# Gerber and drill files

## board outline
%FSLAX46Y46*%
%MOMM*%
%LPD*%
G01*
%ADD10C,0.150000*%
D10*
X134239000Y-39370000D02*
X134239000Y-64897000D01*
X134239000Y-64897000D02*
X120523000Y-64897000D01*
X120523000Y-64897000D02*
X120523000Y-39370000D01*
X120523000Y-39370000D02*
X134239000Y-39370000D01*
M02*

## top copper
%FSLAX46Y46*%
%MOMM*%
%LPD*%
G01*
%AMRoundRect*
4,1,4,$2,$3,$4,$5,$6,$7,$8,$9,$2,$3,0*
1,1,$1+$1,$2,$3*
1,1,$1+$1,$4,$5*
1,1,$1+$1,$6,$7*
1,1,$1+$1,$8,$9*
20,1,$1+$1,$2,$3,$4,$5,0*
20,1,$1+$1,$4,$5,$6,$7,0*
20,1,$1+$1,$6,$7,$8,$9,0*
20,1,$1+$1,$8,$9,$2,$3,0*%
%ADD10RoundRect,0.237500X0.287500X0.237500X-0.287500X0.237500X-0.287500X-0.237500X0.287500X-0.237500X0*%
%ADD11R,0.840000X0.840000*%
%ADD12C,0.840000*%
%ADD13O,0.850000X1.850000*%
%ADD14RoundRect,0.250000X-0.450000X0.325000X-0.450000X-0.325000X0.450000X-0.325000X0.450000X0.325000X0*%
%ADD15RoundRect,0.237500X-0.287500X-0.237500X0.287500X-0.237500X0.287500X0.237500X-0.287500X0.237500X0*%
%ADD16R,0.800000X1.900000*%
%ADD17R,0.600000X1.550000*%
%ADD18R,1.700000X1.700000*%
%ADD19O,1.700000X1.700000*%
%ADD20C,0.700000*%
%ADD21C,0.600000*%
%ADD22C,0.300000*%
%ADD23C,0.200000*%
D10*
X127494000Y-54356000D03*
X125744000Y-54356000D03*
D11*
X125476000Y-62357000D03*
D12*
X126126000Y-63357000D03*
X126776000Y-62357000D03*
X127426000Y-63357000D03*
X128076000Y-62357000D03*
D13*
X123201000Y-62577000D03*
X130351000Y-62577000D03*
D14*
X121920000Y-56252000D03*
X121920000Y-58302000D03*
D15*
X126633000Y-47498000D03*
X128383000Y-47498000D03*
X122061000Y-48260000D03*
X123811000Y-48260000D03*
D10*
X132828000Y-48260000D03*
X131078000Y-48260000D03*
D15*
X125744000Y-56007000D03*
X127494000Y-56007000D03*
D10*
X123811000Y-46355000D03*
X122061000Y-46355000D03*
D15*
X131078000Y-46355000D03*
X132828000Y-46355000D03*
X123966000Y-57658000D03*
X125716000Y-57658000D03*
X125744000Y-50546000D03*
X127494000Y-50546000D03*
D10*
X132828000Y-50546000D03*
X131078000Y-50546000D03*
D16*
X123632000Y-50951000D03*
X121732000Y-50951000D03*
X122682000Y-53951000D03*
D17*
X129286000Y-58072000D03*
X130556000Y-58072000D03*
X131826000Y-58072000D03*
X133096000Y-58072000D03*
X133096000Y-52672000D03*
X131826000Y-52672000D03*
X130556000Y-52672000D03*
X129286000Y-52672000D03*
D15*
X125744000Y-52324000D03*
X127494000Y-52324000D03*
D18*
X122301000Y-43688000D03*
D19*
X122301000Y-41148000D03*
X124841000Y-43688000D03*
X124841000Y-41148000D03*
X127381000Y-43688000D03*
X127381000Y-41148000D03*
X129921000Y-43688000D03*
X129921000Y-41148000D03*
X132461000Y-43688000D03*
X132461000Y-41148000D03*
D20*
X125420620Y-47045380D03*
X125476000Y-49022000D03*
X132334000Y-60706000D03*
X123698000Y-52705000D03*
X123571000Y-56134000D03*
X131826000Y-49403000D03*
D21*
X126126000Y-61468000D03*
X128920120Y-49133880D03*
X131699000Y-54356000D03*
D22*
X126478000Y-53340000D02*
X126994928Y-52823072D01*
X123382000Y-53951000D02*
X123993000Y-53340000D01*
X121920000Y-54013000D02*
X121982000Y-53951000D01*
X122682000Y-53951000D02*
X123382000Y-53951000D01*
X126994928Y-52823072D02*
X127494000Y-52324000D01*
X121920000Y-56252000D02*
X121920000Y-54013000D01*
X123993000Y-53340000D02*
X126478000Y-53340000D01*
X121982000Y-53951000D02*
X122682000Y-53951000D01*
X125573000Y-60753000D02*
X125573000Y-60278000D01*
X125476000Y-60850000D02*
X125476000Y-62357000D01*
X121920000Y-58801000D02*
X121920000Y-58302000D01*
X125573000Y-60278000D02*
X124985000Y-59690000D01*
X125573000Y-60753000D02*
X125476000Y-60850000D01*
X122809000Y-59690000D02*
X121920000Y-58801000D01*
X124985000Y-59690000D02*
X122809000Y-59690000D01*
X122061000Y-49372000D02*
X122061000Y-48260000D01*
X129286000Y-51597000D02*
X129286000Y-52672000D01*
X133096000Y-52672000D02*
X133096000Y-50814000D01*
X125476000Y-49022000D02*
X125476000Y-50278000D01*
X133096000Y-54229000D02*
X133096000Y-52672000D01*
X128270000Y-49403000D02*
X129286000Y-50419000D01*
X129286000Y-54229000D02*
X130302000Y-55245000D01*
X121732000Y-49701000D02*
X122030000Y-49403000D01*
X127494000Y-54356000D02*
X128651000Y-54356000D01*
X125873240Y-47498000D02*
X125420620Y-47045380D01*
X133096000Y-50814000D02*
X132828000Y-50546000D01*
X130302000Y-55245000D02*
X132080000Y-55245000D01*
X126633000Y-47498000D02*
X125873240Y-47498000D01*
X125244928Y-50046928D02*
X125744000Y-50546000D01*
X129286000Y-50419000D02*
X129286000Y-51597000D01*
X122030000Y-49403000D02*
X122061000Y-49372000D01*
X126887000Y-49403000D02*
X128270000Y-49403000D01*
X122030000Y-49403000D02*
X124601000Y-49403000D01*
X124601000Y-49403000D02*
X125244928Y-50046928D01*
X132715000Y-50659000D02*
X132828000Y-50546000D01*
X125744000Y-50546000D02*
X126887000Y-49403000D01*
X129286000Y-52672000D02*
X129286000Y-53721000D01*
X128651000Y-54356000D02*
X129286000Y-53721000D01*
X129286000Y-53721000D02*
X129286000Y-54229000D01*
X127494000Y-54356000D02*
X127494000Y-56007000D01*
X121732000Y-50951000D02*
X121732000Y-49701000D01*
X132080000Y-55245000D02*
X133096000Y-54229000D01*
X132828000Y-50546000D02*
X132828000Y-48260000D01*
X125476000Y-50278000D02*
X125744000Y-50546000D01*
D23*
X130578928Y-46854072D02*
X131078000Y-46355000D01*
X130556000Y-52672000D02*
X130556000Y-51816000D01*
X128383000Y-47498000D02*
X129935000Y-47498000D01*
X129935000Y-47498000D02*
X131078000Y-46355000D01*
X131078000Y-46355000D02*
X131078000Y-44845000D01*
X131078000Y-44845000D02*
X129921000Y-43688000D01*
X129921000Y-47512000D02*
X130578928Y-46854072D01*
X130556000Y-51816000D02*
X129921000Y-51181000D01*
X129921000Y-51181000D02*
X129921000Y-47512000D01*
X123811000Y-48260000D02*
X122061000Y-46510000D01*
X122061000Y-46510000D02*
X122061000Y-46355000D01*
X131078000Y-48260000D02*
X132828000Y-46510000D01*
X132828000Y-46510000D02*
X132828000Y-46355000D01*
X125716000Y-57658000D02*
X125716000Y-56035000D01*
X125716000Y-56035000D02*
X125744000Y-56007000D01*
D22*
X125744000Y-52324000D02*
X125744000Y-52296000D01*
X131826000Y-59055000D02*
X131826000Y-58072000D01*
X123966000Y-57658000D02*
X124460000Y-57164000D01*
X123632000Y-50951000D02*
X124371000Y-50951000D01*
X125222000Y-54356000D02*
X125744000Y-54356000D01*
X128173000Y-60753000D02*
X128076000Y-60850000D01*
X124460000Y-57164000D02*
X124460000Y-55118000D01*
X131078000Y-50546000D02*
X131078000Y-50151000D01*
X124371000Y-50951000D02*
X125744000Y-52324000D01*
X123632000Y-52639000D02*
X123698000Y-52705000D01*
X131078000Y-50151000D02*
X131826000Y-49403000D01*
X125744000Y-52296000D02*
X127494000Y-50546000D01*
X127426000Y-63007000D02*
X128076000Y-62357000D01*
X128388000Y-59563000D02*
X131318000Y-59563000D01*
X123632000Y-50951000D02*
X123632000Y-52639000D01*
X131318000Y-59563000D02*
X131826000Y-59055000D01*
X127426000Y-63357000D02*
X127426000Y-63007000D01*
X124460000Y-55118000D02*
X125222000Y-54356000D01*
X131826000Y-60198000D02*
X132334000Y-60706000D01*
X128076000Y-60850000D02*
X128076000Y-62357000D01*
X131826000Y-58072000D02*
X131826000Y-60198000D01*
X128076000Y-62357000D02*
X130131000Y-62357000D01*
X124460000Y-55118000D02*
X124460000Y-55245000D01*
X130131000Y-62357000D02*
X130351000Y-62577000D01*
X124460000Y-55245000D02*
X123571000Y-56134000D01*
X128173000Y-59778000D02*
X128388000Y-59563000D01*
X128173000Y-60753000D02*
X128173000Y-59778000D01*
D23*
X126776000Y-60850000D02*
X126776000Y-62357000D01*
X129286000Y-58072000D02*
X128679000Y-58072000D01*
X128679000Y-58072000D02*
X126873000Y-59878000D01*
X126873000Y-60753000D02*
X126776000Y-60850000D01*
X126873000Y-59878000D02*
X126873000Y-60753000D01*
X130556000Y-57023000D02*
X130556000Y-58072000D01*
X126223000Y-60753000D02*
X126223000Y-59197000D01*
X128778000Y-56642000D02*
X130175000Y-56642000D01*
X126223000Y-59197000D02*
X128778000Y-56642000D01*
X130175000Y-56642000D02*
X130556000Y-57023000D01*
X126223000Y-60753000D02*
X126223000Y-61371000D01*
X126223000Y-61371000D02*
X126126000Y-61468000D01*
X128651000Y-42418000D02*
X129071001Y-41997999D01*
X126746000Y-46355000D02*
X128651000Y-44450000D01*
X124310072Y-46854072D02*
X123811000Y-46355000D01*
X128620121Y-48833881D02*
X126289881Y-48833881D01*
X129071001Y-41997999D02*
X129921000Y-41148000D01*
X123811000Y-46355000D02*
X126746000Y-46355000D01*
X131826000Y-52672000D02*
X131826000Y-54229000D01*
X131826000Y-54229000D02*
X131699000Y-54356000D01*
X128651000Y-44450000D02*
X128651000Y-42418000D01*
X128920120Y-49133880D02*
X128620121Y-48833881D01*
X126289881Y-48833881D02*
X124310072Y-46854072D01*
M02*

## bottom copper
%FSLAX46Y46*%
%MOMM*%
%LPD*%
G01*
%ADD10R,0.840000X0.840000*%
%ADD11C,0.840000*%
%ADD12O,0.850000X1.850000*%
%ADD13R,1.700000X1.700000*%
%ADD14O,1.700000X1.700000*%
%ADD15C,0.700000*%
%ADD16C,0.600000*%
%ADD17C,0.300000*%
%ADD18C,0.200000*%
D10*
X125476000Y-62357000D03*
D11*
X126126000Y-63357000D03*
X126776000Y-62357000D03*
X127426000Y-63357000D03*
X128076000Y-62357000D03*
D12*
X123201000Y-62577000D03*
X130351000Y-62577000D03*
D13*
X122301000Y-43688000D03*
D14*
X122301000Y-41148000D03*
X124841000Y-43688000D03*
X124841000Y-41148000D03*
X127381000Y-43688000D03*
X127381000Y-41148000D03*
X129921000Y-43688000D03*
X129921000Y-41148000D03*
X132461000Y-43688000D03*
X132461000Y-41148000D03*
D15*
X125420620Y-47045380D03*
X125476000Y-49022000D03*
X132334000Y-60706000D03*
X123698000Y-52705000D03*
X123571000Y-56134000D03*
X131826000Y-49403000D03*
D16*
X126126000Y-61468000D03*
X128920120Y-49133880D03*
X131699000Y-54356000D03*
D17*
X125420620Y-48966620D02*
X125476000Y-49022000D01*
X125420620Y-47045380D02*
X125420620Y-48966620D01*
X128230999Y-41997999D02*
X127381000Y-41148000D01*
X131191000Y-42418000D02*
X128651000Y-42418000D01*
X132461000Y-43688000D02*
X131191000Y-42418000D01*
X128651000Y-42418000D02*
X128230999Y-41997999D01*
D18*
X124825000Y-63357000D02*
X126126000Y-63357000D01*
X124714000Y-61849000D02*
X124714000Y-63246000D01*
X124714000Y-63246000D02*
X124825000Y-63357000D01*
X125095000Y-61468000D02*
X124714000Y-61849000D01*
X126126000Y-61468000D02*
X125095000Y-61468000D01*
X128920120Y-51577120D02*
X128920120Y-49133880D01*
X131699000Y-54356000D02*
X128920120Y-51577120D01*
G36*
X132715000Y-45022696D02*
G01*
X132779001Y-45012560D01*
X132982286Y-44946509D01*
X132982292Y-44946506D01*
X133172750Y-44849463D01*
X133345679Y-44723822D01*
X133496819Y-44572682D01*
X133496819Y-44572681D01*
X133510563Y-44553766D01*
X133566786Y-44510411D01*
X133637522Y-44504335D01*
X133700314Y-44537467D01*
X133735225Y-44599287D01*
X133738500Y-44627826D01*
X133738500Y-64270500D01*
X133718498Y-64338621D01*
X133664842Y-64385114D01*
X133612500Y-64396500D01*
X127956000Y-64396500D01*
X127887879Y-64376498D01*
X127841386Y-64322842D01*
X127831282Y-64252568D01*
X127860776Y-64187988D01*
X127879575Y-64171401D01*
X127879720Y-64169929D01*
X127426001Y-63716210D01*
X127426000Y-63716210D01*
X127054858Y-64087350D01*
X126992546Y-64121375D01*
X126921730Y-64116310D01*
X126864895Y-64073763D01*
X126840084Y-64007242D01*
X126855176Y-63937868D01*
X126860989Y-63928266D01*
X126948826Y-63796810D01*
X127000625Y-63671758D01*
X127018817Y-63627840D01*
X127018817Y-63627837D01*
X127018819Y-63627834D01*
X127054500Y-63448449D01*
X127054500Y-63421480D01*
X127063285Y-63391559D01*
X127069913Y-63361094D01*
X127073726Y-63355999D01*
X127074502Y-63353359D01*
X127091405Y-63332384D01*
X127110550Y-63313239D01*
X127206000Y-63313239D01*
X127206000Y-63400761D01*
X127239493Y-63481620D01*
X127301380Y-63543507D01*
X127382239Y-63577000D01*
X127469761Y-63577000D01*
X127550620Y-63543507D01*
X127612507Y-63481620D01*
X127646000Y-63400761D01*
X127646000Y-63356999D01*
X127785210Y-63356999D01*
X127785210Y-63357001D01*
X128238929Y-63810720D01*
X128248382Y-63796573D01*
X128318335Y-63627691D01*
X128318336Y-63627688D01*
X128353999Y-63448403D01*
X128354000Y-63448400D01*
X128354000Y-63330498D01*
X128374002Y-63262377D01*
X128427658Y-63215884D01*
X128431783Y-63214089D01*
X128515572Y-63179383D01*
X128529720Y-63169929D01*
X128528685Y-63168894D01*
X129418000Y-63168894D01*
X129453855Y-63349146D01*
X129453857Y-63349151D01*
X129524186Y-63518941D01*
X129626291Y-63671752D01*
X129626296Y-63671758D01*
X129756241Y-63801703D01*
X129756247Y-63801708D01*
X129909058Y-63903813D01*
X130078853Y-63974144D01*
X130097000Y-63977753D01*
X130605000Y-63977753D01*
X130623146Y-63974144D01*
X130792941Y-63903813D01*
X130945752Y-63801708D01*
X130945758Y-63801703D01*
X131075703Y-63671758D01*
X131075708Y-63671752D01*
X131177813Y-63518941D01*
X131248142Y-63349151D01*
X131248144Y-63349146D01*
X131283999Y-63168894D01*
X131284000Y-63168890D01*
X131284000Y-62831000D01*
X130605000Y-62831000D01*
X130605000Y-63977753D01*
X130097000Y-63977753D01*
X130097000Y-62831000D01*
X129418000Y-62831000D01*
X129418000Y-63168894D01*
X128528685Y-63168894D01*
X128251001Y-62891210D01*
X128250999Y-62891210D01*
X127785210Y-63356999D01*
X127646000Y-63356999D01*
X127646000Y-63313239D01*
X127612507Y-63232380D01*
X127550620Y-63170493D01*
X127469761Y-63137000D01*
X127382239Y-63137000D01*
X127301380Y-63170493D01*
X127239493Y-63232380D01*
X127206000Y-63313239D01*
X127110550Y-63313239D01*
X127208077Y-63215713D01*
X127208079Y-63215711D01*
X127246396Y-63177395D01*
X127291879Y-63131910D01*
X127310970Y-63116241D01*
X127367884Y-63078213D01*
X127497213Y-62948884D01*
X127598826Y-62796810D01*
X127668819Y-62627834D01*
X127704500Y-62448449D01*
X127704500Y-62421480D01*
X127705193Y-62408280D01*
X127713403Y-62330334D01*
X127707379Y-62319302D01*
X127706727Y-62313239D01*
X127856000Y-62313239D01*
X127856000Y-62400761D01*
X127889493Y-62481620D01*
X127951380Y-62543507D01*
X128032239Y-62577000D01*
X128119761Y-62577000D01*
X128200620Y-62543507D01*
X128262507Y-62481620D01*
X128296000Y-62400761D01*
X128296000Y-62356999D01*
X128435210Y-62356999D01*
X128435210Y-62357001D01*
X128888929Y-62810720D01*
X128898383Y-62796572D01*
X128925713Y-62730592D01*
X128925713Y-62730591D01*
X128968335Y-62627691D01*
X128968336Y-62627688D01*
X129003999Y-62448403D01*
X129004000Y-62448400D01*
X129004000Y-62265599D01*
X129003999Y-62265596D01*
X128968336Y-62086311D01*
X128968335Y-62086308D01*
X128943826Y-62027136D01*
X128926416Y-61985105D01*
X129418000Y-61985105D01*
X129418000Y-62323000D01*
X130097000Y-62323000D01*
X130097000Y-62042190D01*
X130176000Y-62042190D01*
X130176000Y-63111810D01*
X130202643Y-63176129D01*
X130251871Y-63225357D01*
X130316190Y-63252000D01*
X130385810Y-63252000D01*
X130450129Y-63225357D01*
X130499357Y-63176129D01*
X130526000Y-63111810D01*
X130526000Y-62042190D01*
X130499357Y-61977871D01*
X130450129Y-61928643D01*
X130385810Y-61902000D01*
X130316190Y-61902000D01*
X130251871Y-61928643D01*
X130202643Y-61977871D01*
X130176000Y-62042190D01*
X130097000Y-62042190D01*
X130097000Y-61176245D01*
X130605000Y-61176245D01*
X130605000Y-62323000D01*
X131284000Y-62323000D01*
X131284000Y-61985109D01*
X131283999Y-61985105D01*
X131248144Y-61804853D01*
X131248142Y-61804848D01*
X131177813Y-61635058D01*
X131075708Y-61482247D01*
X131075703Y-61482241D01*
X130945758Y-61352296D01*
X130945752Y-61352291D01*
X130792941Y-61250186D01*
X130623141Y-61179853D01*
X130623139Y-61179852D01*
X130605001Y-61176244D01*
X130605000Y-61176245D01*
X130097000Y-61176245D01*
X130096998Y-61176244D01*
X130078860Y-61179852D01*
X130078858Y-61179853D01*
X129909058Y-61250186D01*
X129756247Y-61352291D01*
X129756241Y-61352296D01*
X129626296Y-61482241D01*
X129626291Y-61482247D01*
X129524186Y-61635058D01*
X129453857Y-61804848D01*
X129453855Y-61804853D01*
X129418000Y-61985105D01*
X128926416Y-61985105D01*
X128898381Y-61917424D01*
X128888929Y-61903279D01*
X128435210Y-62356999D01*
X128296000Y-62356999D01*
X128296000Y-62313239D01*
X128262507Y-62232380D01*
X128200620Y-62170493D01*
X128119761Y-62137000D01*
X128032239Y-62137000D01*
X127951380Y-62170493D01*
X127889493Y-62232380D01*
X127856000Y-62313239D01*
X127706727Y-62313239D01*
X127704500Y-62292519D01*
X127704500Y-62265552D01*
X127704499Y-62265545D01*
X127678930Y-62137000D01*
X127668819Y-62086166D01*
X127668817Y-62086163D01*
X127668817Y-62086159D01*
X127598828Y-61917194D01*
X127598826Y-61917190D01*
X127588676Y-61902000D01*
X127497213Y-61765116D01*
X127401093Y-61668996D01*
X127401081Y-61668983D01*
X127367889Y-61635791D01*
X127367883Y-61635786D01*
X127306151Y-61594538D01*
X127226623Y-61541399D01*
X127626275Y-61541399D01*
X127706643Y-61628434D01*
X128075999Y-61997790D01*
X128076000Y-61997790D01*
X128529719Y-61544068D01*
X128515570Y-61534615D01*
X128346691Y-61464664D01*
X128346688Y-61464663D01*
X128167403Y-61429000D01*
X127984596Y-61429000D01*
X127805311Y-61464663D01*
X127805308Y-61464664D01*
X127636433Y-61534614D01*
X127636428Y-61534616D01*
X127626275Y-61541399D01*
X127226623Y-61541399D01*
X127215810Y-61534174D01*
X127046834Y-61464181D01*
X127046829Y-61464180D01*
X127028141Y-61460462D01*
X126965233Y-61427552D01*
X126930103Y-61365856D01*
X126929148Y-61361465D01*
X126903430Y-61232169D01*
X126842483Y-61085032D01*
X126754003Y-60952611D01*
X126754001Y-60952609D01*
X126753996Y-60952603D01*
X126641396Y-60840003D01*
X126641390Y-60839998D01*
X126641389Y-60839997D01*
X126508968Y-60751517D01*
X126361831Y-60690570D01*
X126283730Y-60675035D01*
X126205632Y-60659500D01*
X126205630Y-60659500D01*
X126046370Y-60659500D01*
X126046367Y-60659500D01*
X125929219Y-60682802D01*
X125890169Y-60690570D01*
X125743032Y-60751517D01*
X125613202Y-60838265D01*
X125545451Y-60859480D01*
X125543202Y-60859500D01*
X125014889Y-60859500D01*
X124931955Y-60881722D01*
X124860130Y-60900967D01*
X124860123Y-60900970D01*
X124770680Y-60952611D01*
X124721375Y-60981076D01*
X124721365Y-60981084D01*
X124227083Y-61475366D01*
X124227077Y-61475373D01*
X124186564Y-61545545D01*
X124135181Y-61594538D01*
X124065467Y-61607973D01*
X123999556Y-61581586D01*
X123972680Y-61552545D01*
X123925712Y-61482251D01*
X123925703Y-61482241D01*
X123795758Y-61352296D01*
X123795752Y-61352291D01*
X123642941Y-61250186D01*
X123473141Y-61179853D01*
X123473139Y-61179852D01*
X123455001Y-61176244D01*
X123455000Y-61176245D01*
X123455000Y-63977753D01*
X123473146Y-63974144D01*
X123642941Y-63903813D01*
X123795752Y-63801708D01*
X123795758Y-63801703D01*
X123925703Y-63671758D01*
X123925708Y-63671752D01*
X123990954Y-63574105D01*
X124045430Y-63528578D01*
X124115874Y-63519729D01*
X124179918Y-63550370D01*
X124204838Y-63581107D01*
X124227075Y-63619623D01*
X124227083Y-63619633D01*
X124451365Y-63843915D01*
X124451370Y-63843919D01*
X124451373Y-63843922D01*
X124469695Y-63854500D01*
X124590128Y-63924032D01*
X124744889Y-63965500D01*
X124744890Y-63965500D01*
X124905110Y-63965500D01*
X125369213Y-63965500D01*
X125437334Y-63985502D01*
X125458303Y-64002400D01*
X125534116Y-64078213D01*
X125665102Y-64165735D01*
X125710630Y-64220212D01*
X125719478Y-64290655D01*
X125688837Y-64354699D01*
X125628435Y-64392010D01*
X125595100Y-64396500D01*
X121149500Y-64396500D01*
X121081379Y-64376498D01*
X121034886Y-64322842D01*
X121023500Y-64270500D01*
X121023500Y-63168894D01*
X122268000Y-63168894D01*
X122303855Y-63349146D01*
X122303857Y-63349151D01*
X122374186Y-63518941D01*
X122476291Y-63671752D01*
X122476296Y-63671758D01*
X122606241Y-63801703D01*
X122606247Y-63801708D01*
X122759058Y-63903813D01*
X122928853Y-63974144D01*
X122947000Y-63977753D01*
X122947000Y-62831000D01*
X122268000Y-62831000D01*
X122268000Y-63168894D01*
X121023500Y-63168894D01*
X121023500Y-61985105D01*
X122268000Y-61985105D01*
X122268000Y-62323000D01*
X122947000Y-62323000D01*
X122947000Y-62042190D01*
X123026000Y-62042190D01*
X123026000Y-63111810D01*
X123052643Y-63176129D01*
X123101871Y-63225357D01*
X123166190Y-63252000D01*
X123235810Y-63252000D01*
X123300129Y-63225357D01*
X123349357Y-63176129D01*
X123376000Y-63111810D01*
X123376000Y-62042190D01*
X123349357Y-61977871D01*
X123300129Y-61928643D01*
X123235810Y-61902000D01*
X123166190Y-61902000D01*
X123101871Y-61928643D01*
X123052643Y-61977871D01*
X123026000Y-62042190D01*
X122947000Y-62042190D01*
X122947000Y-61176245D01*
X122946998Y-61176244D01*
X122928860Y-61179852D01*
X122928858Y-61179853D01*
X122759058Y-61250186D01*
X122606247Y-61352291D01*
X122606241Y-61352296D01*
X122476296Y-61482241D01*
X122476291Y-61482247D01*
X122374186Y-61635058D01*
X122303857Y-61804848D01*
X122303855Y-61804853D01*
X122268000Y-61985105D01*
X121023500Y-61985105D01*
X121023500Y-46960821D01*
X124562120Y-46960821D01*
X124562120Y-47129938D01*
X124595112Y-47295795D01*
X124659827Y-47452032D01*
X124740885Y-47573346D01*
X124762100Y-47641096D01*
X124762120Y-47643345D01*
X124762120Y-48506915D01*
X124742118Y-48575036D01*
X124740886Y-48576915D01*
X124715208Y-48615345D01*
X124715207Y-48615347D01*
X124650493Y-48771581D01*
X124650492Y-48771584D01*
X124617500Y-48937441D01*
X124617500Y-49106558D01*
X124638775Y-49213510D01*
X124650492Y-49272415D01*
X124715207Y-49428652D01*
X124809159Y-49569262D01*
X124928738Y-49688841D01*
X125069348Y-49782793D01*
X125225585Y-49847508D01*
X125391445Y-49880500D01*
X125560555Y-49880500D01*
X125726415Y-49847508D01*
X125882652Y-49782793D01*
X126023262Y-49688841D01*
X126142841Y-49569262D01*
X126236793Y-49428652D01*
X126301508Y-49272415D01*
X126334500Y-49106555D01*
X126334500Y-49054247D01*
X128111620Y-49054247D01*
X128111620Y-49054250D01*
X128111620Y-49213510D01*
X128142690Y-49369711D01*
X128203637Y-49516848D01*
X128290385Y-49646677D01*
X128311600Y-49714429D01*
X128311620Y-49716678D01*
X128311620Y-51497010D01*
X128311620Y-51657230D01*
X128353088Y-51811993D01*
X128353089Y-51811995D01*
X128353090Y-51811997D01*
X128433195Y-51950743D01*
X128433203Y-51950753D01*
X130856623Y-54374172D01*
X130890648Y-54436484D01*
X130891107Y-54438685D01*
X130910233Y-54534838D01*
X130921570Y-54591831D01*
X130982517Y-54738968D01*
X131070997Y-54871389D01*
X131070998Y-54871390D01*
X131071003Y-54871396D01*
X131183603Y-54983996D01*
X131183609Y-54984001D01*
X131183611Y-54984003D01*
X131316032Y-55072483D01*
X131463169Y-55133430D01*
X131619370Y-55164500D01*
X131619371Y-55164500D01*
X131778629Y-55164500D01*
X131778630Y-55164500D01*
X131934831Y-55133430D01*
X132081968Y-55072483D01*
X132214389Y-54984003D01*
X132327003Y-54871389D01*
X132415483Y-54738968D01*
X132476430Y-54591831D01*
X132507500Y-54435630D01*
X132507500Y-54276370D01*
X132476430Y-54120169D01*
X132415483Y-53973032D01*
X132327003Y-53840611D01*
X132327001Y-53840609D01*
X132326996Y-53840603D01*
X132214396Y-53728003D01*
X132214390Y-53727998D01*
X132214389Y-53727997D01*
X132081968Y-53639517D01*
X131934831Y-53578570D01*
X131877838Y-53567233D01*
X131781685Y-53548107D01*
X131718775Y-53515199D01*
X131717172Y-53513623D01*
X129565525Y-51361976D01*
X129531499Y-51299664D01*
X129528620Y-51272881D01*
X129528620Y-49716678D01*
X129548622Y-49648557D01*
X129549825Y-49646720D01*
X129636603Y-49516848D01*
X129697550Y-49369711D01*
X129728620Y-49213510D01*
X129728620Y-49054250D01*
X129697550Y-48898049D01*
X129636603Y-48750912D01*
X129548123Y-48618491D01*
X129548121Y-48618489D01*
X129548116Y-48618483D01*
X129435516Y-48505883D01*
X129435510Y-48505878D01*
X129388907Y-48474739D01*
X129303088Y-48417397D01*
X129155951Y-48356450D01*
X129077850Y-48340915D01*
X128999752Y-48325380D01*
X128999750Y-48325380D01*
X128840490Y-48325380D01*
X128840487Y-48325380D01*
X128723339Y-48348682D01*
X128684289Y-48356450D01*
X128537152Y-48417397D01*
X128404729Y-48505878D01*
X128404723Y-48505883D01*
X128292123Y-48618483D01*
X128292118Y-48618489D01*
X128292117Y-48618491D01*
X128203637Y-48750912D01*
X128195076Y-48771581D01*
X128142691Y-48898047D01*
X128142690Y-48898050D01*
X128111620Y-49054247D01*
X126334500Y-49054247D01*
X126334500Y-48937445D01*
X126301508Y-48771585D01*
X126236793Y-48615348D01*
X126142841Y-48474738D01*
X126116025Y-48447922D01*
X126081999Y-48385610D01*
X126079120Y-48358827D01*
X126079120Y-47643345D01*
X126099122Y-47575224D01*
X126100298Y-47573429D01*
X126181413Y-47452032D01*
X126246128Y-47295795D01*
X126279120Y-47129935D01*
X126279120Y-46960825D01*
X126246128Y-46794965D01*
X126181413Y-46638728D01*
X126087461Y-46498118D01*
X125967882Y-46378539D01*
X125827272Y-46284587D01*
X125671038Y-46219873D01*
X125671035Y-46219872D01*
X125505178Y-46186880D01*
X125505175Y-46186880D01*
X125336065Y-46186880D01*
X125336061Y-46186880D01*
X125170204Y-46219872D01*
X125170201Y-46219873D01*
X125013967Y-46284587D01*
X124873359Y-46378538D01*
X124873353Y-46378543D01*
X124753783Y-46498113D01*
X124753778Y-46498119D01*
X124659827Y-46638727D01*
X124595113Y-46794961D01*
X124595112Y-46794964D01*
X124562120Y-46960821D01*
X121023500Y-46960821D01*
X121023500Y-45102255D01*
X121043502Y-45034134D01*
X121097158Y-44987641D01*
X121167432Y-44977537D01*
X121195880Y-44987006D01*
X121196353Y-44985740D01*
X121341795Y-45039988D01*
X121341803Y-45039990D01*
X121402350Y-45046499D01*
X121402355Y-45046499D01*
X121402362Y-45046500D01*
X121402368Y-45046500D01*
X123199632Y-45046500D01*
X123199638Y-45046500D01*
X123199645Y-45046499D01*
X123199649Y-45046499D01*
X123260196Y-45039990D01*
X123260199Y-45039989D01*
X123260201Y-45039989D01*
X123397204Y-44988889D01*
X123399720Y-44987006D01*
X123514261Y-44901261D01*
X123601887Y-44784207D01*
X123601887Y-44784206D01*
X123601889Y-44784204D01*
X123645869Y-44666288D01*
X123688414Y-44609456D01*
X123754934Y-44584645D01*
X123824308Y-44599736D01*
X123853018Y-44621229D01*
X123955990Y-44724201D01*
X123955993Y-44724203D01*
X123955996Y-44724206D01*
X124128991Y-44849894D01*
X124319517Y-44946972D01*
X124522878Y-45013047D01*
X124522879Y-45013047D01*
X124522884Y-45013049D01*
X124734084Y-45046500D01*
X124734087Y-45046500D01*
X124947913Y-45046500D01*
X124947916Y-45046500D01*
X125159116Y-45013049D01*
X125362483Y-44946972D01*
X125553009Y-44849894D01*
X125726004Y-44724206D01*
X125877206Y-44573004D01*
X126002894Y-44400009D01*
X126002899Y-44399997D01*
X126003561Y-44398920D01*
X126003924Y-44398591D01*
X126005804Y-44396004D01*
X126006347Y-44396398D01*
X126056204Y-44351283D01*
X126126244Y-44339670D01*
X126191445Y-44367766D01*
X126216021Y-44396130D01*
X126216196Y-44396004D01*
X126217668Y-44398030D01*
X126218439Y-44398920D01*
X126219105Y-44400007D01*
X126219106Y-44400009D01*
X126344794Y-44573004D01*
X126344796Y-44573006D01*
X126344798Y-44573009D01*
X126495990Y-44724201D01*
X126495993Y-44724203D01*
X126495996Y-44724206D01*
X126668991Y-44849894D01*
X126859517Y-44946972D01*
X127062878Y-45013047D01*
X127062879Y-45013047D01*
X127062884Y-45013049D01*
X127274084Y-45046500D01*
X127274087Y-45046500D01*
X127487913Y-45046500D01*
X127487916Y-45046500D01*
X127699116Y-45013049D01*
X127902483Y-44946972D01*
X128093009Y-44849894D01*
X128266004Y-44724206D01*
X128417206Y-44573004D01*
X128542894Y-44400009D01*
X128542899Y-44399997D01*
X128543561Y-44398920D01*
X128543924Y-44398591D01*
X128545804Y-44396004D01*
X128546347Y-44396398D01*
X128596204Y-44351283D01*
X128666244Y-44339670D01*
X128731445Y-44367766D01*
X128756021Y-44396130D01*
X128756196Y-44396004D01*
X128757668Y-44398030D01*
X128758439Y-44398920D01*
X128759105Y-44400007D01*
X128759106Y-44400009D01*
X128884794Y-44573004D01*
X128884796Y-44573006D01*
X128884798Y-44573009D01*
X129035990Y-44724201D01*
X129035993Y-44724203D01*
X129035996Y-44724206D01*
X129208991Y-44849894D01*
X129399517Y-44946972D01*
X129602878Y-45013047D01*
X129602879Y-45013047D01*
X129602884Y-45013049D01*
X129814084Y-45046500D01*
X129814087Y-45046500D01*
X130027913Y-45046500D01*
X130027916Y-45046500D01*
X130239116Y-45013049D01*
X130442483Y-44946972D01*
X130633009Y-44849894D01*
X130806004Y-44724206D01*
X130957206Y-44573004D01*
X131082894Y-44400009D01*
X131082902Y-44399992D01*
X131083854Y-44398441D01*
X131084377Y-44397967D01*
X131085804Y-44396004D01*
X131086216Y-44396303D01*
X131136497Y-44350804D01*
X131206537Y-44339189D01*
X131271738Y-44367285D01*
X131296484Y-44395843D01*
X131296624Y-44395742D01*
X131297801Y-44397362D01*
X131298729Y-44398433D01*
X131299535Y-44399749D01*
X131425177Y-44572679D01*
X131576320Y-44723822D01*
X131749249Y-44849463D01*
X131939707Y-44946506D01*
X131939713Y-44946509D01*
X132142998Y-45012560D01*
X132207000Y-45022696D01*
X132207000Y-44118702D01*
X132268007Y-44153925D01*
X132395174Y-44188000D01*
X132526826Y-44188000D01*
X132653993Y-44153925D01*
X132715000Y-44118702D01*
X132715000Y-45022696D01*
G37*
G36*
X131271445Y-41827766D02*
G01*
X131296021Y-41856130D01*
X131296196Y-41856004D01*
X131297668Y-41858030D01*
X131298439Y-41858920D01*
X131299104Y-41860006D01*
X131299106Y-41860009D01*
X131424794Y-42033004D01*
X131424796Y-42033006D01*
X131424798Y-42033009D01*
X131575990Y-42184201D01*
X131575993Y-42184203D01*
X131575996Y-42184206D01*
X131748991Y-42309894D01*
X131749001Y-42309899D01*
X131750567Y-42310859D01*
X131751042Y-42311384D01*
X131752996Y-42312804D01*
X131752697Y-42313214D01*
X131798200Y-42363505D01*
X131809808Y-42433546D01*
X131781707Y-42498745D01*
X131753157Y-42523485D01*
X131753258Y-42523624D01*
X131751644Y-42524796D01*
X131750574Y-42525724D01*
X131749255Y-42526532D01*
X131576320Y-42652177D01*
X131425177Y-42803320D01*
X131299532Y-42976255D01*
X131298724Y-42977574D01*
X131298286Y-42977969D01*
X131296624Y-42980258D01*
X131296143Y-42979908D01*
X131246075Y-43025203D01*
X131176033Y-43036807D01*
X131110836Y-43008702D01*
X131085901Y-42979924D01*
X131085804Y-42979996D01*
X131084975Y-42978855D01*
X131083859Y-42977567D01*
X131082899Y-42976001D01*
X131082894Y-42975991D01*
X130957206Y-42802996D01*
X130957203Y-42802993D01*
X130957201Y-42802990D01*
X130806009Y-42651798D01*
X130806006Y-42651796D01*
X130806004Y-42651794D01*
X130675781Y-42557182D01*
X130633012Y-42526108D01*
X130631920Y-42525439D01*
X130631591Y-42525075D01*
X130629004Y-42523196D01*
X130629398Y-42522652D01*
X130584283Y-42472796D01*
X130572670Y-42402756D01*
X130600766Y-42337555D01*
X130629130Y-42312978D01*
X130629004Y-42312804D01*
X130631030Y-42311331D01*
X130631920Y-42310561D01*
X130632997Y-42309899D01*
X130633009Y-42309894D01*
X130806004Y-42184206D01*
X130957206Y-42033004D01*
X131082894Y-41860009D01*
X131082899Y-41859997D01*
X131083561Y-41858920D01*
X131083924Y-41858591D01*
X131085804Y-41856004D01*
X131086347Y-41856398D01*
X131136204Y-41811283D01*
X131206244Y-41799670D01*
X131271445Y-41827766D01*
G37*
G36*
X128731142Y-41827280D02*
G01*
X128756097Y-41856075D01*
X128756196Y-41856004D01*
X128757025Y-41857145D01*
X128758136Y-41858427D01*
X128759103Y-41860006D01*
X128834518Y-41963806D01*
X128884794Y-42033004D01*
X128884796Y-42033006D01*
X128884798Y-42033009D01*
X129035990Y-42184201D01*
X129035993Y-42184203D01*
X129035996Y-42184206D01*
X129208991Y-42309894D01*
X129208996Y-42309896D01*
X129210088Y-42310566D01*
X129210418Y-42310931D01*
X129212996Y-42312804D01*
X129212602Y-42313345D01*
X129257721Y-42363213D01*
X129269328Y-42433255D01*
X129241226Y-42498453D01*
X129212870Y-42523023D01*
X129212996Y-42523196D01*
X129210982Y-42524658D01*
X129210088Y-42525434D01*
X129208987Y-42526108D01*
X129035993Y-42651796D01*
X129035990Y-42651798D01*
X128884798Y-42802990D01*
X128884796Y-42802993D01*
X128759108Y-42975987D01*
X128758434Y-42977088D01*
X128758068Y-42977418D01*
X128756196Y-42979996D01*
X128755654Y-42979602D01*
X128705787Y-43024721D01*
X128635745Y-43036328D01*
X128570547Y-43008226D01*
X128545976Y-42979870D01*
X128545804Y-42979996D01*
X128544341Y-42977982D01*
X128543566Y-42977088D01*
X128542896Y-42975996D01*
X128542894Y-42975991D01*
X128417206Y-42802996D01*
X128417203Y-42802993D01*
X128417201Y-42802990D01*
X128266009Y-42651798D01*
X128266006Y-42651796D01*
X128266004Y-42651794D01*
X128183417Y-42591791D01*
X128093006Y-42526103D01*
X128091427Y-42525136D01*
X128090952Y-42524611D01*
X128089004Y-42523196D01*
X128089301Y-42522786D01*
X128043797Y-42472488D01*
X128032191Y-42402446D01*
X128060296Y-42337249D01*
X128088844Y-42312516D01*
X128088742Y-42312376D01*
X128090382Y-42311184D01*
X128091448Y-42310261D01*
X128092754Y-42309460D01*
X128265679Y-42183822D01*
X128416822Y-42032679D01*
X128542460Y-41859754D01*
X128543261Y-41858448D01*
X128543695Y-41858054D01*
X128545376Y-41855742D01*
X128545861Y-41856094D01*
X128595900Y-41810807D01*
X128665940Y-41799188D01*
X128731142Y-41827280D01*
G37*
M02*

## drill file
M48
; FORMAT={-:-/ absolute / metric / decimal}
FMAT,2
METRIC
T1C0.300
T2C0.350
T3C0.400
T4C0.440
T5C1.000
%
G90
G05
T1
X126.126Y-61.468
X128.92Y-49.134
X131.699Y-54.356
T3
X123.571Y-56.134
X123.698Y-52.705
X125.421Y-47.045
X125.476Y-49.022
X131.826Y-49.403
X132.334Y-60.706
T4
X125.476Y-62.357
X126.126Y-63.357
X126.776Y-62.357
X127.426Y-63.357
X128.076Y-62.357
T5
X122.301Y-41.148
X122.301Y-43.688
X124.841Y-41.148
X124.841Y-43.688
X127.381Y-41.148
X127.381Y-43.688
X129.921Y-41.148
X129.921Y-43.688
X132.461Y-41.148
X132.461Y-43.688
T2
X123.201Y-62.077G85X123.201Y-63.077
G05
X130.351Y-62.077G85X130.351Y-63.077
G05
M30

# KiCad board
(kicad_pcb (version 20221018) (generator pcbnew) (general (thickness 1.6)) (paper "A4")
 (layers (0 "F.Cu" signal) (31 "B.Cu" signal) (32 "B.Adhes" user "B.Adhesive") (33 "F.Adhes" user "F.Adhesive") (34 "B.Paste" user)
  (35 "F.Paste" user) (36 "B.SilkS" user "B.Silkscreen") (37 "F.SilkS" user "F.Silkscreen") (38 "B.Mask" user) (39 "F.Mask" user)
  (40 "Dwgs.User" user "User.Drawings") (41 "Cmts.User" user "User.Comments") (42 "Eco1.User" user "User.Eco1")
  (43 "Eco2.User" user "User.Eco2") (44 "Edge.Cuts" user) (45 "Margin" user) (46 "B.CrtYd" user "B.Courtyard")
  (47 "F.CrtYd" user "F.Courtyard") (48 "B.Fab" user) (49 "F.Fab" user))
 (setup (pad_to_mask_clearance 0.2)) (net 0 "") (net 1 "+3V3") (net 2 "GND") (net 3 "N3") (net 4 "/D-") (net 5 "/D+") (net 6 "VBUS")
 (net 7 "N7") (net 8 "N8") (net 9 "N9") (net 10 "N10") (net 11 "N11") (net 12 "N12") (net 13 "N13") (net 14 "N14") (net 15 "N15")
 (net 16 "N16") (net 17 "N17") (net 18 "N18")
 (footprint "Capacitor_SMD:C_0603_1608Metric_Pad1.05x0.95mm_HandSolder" (layer "F.Cu") (at 126.619 54.356 180)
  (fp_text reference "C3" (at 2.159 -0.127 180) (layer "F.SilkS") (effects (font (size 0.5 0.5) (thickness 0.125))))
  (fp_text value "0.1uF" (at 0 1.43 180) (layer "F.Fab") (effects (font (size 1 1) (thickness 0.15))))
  (pad "1" smd roundrect (at -0.875 0 180) (size 1.05 0.95) (layers "F.Cu" "F.Paste" "F.Mask") (roundrect_rratio 0.25) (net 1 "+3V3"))
  (pad "2" smd roundrect (at 0.875 0 180) (size 1.05 0.95) (layers "F.Cu" "F.Paste" "F.Mask") (roundrect_rratio 0.25) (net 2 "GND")))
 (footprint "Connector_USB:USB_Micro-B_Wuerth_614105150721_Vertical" (layer "F.Cu") (at 125.476 62.357)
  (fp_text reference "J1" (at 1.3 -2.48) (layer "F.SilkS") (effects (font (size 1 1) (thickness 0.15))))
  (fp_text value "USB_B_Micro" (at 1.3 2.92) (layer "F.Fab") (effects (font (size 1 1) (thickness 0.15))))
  (pad "1" thru_hole rect (at 0 0) (size 0.84 0.84) (drill 0.44) (layers "*.Cu" "*.Mask") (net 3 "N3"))
  (pad "2" thru_hole circle (at 0.65 1) (size 0.84 0.84) (drill 0.44) (layers "*.Cu" "*.Mask") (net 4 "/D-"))
  (pad "3" thru_hole circle (at 1.3 0) (size 0.84 0.84) (drill 0.44) (layers "*.Cu" "*.Mask") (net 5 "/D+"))
  (pad "4" thru_hole circle (at 1.95 1) (size 0.84 0.84) (drill 0.44) (layers "*.Cu" "*.Mask") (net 2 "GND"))
  (pad "5" thru_hole circle (at 2.6 0) (size 0.84 0.84) (drill 0.44) (layers "*.Cu" "*.Mask") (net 2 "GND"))
  (pad "6" thru_hole oval (at -2.275 0.22) (size 0.85 1.85) (drill oval 0.35 1.35) (layers "*.Cu" "*.Mask") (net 2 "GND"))
  (pad "6" thru_hole oval (at 4.875 0.22) (size 0.85 1.85) (drill oval 0.35 1.35) (layers "*.Cu" "*.Mask") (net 2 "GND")))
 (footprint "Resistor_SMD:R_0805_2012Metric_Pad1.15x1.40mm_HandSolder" (layer "F.Cu") (at 121.92 57.277 -90)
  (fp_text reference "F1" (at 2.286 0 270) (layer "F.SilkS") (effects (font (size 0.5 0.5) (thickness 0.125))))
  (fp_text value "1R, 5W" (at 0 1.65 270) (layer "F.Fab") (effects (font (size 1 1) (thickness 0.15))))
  (pad "1" smd roundrect (at -1.025 0 270) (size 1.15 1.4) (layers "F.Cu" "F.Paste" "F.Mask") (roundrect_rratio 0.217391) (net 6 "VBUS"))
  (pad "2" smd roundrect (at 1.025 0 270) (size 1.15 1.4) (layers "F.Cu" "F.Paste" "F.Mask") (roundrect_rratio 0.217391) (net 3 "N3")))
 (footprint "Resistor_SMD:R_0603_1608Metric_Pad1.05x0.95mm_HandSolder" (layer "F.Cu") (at 127.508 47.498)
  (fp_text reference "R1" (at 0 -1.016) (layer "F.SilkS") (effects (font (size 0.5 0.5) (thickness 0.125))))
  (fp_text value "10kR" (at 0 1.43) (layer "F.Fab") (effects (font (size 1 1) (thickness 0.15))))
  (pad "1" smd roundrect (at -0.875 0) (size 1.05 0.95) (layers "F.Cu" "F.Paste" "F.Mask") (roundrect_rratio 0.25) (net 1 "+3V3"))
  (pad "2" smd roundrect (at 0.875 0) (size 1.05 0.95) (layers "F.Cu" "F.Paste" "F.Mask") (roundrect_rratio 0.25) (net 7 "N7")))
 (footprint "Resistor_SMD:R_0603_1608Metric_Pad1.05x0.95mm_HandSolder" (layer "F.Cu") (at 122.936 48.26)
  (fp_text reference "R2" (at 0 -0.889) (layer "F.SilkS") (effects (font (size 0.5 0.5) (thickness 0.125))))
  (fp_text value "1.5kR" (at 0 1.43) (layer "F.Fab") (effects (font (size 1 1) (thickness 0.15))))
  (pad "1" smd roundrect (at -0.875 0) (size 1.05 0.95) (layers "F.Cu" "F.Paste" "F.Mask") (roundrect_rratio 0.25) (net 1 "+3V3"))
  (pad "2" smd roundrect (at 0.875 0) (size 1.05 0.95) (layers "F.Cu" "F.Paste" "F.Mask") (roundrect_rratio 0.25) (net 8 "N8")))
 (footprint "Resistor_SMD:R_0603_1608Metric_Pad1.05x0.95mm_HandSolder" (layer "F.Cu") (at 131.953 48.26 180)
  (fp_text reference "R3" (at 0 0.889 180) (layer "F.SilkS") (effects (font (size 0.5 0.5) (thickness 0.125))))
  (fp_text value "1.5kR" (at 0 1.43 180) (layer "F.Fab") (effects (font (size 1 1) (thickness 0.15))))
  (pad "1" smd roundrect (at -0.875 0 180) (size 1.05 0.95) (layers "F.Cu" "F.Paste" "F.Mask") (roundrect_rratio 0.25) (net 1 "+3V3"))
  (pad "2" smd roundrect (at 0.875 0 180) (size 1.05 0.95) (layers "F.Cu" "F.Paste" "F.Mask") (roundrect_rratio 0.25) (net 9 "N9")))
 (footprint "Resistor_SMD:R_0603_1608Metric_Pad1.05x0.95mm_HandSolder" (layer "F.Cu") (at 126.619 56.007)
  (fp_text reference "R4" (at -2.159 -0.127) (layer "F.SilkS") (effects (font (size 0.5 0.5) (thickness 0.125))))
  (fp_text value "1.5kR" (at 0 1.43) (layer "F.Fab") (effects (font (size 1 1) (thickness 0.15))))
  (pad "1" smd roundrect (at -0.875 0) (size 1.05 0.95) (layers "F.Cu" "F.Paste" "F.Mask") (roundrect_rratio 0.25) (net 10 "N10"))
  (pad "2" smd roundrect (at 0.875 0) (size 1.05 0.95) (layers "F.Cu" "F.Paste" "F.Mask") (roundrect_rratio 0.25) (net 1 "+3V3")))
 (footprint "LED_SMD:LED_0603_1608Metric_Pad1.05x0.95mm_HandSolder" (layer "F.Cu") (at 122.936 46.355 180)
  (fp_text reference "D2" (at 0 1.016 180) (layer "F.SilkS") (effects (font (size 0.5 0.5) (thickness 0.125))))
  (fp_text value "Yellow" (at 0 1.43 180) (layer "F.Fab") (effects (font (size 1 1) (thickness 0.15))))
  (pad "1" smd roundrect (at -0.875 0 180) (size 1.05 0.95) (layers "F.Cu" "F.Paste" "F.Mask") (roundrect_rratio 0.25) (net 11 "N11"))
  (pad "2" smd roundrect (at 0.875 0 180) (size 1.05 0.95) (layers "F.Cu" "F.Paste" "F.Mask") (roundrect_rratio 0.25) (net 8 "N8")))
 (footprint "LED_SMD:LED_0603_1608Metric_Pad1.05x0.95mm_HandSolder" (layer "F.Cu") (at 131.953 46.355)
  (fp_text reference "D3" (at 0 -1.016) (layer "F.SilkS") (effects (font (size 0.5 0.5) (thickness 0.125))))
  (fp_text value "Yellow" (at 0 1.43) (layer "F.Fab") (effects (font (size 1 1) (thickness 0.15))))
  (pad "1" smd roundrect (at -0.875 0) (size 1.05 0.95) (layers "F.Cu" "F.Paste" "F.Mask") (roundrect_rratio 0.25) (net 7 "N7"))
  (pad "2" smd roundrect (at 0.875 0) (size 1.05 0.95) (layers "F.Cu" "F.Paste" "F.Mask") (roundrect_rratio 0.25) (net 9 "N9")))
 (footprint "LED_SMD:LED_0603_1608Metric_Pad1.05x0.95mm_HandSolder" (layer "F.Cu") (at 124.841 57.658)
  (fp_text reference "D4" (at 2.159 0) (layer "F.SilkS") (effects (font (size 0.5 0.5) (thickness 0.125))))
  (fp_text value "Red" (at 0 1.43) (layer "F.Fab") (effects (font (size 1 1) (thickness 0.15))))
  (pad "1" smd roundrect (at -0.875 0) (size 1.05 0.95) (layers "F.Cu" "F.Paste" "F.Mask") (roundrect_rratio 0.25) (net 2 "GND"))
  (pad "2" smd roundrect (at 0.875 0) (size 1.05 0.95) (layers "F.Cu" "F.Paste" "F.Mask") (roundrect_rratio 0.25) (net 10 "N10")))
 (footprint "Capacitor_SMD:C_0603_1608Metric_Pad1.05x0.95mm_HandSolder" (layer "F.Cu") (at 126.619 50.546)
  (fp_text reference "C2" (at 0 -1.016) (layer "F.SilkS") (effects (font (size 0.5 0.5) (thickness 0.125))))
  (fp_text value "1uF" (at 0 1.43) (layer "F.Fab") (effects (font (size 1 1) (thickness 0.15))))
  (pad "1" smd roundrect (at -0.875 0) (size 1.05 0.95) (layers "F.Cu" "F.Paste" "F.Mask") (roundrect_rratio 0.25) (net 1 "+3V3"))
  (pad "2" smd roundrect (at 0.875 0) (size 1.05 0.95) (layers "F.Cu" "F.Paste" "F.Mask") (roundrect_rratio 0.25) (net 2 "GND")))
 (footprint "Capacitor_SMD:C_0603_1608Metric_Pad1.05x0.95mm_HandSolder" (layer "F.Cu") (at 131.953 50.546 180)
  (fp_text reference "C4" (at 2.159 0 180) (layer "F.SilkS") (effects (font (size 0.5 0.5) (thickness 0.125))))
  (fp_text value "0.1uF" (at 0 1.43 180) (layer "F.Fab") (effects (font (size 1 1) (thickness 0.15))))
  (pad "1" smd roundrect (at -0.875 0 180) (size 1.05 0.95) (layers "F.Cu" "F.Paste" "F.Mask") (roundrect_rratio 0.25) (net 1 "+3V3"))
  (pad "2" smd roundrect (at 0.875 0 180) (size 1.05 0.95) (layers "F.Cu" "F.Paste" "F.Mask") (roundrect_rratio 0.25) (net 2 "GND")))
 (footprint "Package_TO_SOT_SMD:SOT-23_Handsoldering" (layer "F.Cu") (at 122.682 52.451 -90)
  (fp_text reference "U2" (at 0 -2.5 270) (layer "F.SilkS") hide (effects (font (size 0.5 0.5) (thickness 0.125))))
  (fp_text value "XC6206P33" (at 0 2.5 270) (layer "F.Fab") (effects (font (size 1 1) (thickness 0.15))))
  (pad "1" smd rect (at -1.5 -0.95 270) (size 1.9 0.8) (layers "F.Cu" "F.Paste" "F.Mask") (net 2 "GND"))
  (pad "2" smd rect (at -1.5 0.95 270) (size 1.9 0.8) (layers "F.Cu" "F.Paste" "F.Mask") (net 1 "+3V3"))
  (pad "3" smd rect (at 1.5 0 270) (size 1.9 0.8) (layers "F.Cu" "F.Paste" "F.Mask") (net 6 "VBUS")))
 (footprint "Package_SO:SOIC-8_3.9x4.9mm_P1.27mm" (layer "F.Cu") (at 131.191 55.372 90)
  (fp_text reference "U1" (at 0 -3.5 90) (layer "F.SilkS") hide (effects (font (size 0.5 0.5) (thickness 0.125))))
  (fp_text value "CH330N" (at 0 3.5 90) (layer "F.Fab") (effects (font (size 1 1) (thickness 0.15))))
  (pad "1" smd rect (at -2.7 -1.905 90) (size 1.55 0.6) (layers "F.Cu" "F.Paste" "F.Mask") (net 5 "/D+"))
  (pad "2" smd rect (at -2.7 -0.635 90) (size 1.55 0.6) (layers "F.Cu" "F.Paste" "F.Mask") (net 4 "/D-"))
  (pad "3" smd rect (at -2.7 0.635 90) (size 1.55 0.6) (layers "F.Cu" "F.Paste" "F.Mask") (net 2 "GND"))
  (pad "4" smd rect (at -2.7 1.905 90) (size 1.55 0.6) (layers "F.Cu" "F.Paste" "F.Mask") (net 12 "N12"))
  (pad "5" smd rect (at 2.7 1.905 90) (size 1.55 0.6) (layers "F.Cu" "F.Paste" "F.Mask") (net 1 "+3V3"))
  (pad "6" smd rect (at 2.7 0.635 90) (size 1.55 0.6) (layers "F.Cu" "F.Paste" "F.Mask") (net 11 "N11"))
  (pad "7" smd rect (at 2.7 -0.635 90) (size 1.55 0.6) (layers "F.Cu" "F.Paste" "F.Mask") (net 7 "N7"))
  (pad "8" smd rect (at 2.7 -1.905 90) (size 1.55 0.6) (layers "F.Cu" "F.Paste" "F.Mask") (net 1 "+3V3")))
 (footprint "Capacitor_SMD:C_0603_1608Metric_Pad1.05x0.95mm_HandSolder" (layer "F.Cu") (at 126.619 52.324)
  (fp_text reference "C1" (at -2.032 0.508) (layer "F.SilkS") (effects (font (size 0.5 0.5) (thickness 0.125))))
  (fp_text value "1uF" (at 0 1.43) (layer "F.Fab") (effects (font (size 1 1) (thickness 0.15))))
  (pad "1" smd roundrect (at -0.875 0) (size 1.05 0.95) (layers "F.Cu" "F.Paste" "F.Mask") (roundrect_rratio 0.25) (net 2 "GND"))
  (pad "2" smd roundrect (at 0.875 0) (size 1.05 0.95) (layers "F.Cu" "F.Paste" "F.Mask") (roundrect_rratio 0.25) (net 6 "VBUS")))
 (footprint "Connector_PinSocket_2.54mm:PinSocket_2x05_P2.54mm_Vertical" (layer "B.Cu") (at 122.301 43.688 -90)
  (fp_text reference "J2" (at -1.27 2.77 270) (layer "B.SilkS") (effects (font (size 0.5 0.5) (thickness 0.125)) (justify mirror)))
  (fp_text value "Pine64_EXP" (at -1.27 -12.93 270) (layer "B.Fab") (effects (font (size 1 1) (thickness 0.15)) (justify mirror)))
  (pad "1" thru_hole rect (at 0 0 270) (size 1.7 1.7) (drill 1) (layers "*.Cu" "*.Mask") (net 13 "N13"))
  (pad "2" thru_hole oval (at -2.54 0 270) (size 1.7 1.7) (drill 1) (layers "*.Cu" "*.Mask") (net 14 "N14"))
  (pad "3" thru_hole oval (at 0 -2.54 270) (size 1.7 1.7) (drill 1) (layers "*.Cu" "*.Mask") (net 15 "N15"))
  (pad "4" thru_hole oval (at -2.54 -2.54 270) (size 1.7 1.7) (drill 1) (layers "*.Cu" "*.Mask") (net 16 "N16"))
  (pad "5" thru_hole oval (at 0 -5.08 270) (size 1.7 1.7) (drill 1) (layers "*.Cu" "*.Mask") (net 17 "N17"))
  (pad "6" thru_hole oval (at -2.54 -5.08 270) (size 1.7 1.7) (drill 1) (layers "*.Cu" "*.Mask") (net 2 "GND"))
  (pad "7" thru_hole oval (at 0 -7.62 270) (size 1.7 1.7) (drill 1) (layers "*.Cu" "*.Mask") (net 7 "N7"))
  (pad "8" thru_hole oval (at -2.54 -7.62 270) (size 1.7 1.7) (drill 1) (layers "*.Cu" "*.Mask") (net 11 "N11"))
  (pad "9" thru_hole oval (at 0 -10.16 270) (size 1.7 1.7) (drill 1) (layers "*.Cu" "*.Mask") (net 2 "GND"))
  (pad "10" thru_hole oval (at -2.54 -10.16 270) (size 1.7 1.7) (drill 1) (layers "*.Cu" "*.Mask") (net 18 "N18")))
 (gr_line (start 134.239 39.37) (end 134.239 64.897) (stroke (width 0.15) (type solid)) (layer "Edge.Cuts"))
 (gr_line (start 134.239 64.897) (end 120.523 64.897) (stroke (width 0.15) (type solid)) (layer "Edge.Cuts"))
 (gr_line (start 120.523 64.897) (end 120.523 39.37) (stroke (width 0.15) (type solid)) (layer "Edge.Cuts"))
 (gr_line (start 120.523 39.37) (end 134.239 39.37) (stroke (width 0.15) (type solid)) (layer "Edge.Cuts"))
 (segment (start 126.478 53.34) (end 126.994928 52.823072) (width 0.3) (layer "F.Cu") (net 6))
 (segment (start 123.382 53.951) (end 123.993 53.34) (width 0.3) (layer "F.Cu") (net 6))
 (segment (start 121.92 54.013) (end 121.982 53.951) (width 0.3) (layer "F.Cu") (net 6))
 (segment (start 122.682 53.951) (end 123.382 53.951) (width 0.3) (layer "F.Cu") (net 6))
 (segment (start 126.994928 52.823072) (end 127.494 52.324) (width 0.3) (layer "F.Cu") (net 6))
 (segment (start 121.92 56.252) (end 121.92 54.013) (width 0.3) (layer "F.Cu") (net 6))
 (segment (start 123.993 53.34) (end 126.478 53.34) (width 0.3) (layer "F.Cu") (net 6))
 (segment (start 121.982 53.951) (end 122.682 53.951) (width 0.3) (layer "F.Cu") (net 6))
 (segment (start 125.573 60.753) (end 125.573 60.278) (width 0.3) (layer "F.Cu") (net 3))
 (segment (start 125.476 60.85) (end 125.476 62.357) (width 0.3) (layer "F.Cu") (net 3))
 (segment (start 121.92 58.801) (end 121.92 58.302) (width 0.3) (layer "F.Cu") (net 3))
 (segment (start 125.573 60.278) (end 124.985 59.69) (width 0.3) (layer "F.Cu") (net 3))
 (segment (start 125.573 60.753) (end 125.476 60.85) (width 0.3) (layer "F.Cu") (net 3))
 (segment (start 122.809 59.69) (end 121.92 58.801) (width 0.3) (layer "F.Cu") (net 3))
 (segment (start 124.985 59.69) (end 122.809 59.69) (width 0.3) (layer "F.Cu") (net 3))
 (segment (start 122.061 49.372) (end 122.061 48.26) (width 0.3) (layer "F.Cu") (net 1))
 (segment (start 129.286 51.597) (end 129.286 52.672) (width 0.3) (layer "F.Cu") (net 1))
 (segment (start 133.096 52.672) (end 133.096 50.814) (width 0.3) (layer "F.Cu") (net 1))
 (segment (start 125.476 49.022) (end 125.476 50.278) (width 0.3) (layer "F.Cu") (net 1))
 (segment (start 133.096 54.229) (end 133.096 52.672) (width 0.3) (layer "F.Cu") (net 1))
 (segment (start 128.27 49.403) (end 129.286 50.419) (width 0.3) (layer "F.Cu") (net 1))
 (segment (start 129.286 54.229) (end 130.302 55.245) (width 0.3) (layer "F.Cu") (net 1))
 (segment (start 121.732 49.701) (end 122.03 49.403) (width 0.3) (layer "F.Cu") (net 1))
 (segment (start 127.494 54.356) (end 128.651 54.356) (width 0.3) (layer "F.Cu") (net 1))
 (segment (start 125.87324 47.498) (end 125.42062 47.04538) (width 0.3) (layer "F.Cu") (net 1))
 (segment (start 133.096 50.814) (end 132.828 50.546) (width 0.3) (layer "F.Cu") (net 1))
 (segment (start 130.302 55.245) (end 132.08 55.245) (width 0.3) (layer "F.Cu") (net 1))
 (segment (start 126.633 47.498) (end 125.87324 47.498) (width 0.3) (layer "F.Cu") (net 1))
 (segment (start 125.244928 50.046928) (end 125.744 50.546) (width 0.3) (layer "F.Cu") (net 1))
 (segment (start 129.286 50.419) (end 129.286 51.597) (width 0.3) (layer "F.Cu") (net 1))
 (segment (start 122.03 49.403) (end 122.061 49.372) (width 0.3) (layer "F.Cu") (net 1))
 (segment (start 126.887 49.403) (end 128.27 49.403) (width 0.3) (layer "F.Cu") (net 1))
 (segment (start 122.03 49.403) (end 124.601 49.403) (width 0.3) (layer "F.Cu") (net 1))
 (segment (start 124.601 49.403) (end 125.244928 50.046928) (width 0.3) (layer "F.Cu") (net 1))
 (segment (start 132.715 50.659) (end 132.828 50.546) (width 0.3) (layer "F.Cu") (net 1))
 (segment (start 125.744 50.546) (end 126.887 49.403) (width 0.3) (layer "F.Cu") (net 1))
 (segment (start 129.286 52.672) (end 129.286 53.721) (width 0.3) (layer "F.Cu") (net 1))
 (segment (start 128.651 54.356) (end 129.286 53.721) (width 0.3) (layer "F.Cu") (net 1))
 (segment (start 129.286 53.721) (end 129.286 54.229) (width 0.3) (layer "F.Cu") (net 1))
 (segment (start 127.494 54.356) (end 127.494 56.007) (width 0.3) (layer "F.Cu") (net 1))
 (segment (start 121.732 50.951) (end 121.732 49.701) (width 0.3) (layer "F.Cu") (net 1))
 (segment (start 132.08 55.245) (end 133.096 54.229) (width 0.3) (layer "F.Cu") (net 1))
 (segment (start 132.828 50.546) (end 132.828 48.26) (width 0.3) (layer "F.Cu") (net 1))
 (segment (start 125.476 50.278) (end 125.744 50.546) (width 0.3) (layer "F.Cu") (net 1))
 (via (at 125.42062 47.04538) (size 0.7) (drill 0.4) (layers "F.Cu" "B.Cu") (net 1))
 (via (at 125.476 49.022) (size 0.7) (drill 0.4) (layers "F.Cu" "B.Cu") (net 1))
 (segment (start 125.42062 48.96662) (end 125.476 49.022) (width 0.3) (layer "B.Cu") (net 1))
 (segment (start 125.42062 47.04538) (end 125.42062 48.96662) (width 0.3) (layer "B.Cu") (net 1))
 (segment (start 130.578928 46.854072) (end 131.078 46.355) (width 0.2) (layer "F.Cu") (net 7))
 (segment (start 130.556 52.672) (end 130.556 51.816) (width 0.2) (layer "F.Cu") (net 7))
 (segment (start 128.383 47.498) (end 129.935 47.498) (width 0.2) (layer "F.Cu") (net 7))
 (segment (start 129.935 47.498) (end 131.078 46.355) (width 0.2) (layer "F.Cu") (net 7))
 (segment (start 131.078 46.355) (end 131.078 44.845) (width 0.2) (layer "F.Cu") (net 7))
 (segment (start 131.078 44.845) (end 129.921 43.688) (width 0.2) (layer "F.Cu") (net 7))
 (segment (start 129.921 47.512) (end 130.578928 46.854072) (width 0.2) (layer "F.Cu") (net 7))
 (segment (start 130.556 51.816) (end 129.921 51.181) (width 0.2) (layer "F.Cu") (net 7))
 (segment (start 129.921 51.181) (end 129.921 47.512) (width 0.2) (layer "F.Cu") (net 7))
 (segment (start 123.811 48.26) (end 122.061 46.51) (width 0.2) (layer "F.Cu") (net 8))
 (segment (start 122.061 46.51) (end 122.061 46.355) (width 0.2) (layer "F.Cu") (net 8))
 (segment (start 131.078 48.26) (end 132.828 46.51) (width 0.2) (layer "F.Cu") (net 9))
 (segment (start 132.828 46.51) (end 132.828 46.355) (width 0.2) (layer "F.Cu") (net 9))
 (segment (start 125.716 57.658) (end 125.716 56.035) (width 0.2) (layer "F.Cu") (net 10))
 (segment (start 125.716 56.035) (end 125.744 56.007) (width 0.2) (layer "F.Cu") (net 10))
 (segment (start 125.744 52.324) (end 125.744 52.296) (width 0.3) (layer "F.Cu") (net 2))
 (segment (start 131.826 59.055) (end 131.826 58.072) (width 0.3) (layer "F.Cu") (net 2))
 (segment (start 123.966 57.658) (end 124.46 57.164) (width 0.3) (layer "F.Cu") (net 2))
 (segment (start 123.632 50.951) (end 124.371 50.951) (width 0.3) (layer "F.Cu") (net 2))
 (segment (start 125.222 54.356) (end 125.744 54.356) (width 0.3) (layer "F.Cu") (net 2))
 (segment (start 128.173 60.753) (end 128.076 60.85) (width 0.3) (layer "F.Cu") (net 2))
 (segment (start 124.46 57.164) (end 124.46 55.118) (width 0.3) (layer "F.Cu") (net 2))
 (segment (start 131.078 50.546) (end 131.078 50.151) (width 0.3) (layer "F.Cu") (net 2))
 (segment (start 124.371 50.951) (end 125.744 52.324) (width 0.3) (layer "F.Cu") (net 2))
 (segment (start 123.632 52.639) (end 123.698 52.705) (width 0.3) (layer "F.Cu") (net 2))
 (segment (start 131.078 50.151) (end 131.826 49.403) (width 0.3) (layer "F.Cu") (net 2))
 (segment (start 125.744 52.296) (end 127.494 50.546) (width 0.3) (layer "F.Cu") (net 2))
 (segment (start 127.426 63.007) (end 128.076 62.357) (width 0.3) (layer "F.Cu") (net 2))
 (segment (start 128.388 59.563) (end 131.318 59.563) (width 0.3) (layer "F.Cu") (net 2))
 (segment (start 123.632 50.951) (end 123.632 52.639) (width 0.3) (layer "F.Cu") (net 2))
 (segment (start 131.318 59.563) (end 131.826 59.055) (width 0.3) (layer "F.Cu") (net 2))
 (segment (start 127.426 63.357) (end 127.426 63.007) (width 0.3) (layer "F.Cu") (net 2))
 (segment (start 124.46 55.118) (end 125.222 54.356) (width 0.3) (layer "F.Cu") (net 2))
 (segment (start 131.826 60.198) (end 132.334 60.706) (width 0.3) (layer "F.Cu") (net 2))
 (segment (start 128.076 60.85) (end 128.076 62.357) (width 0.3) (layer "F.Cu") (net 2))
 (segment (start 131.826 58.072) (end 131.826 60.198) (width 0.3) (layer "F.Cu") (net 2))
 (segment (start 128.076 62.357) (end 130.131 62.357) (width 0.3) (layer "F.Cu") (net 2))
 (segment (start 124.46 55.118) (end 124.46 55.245) (width 0.3) (layer "F.Cu") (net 2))
 (segment (start 130.131 62.357) (end 130.351 62.577) (width 0.3) (layer "F.Cu") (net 2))
 (segment (start 124.46 55.245) (end 123.571 56.134) (width 0.3) (layer "F.Cu") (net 2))
 (segment (start 128.173 59.778) (end 128.388 59.563) (width 0.3) (layer "F.Cu") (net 2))
 (segment (start 128.173 60.753) (end 128.173 59.778) (width 0.3) (layer "F.Cu") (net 2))
 (via (at 132.334 60.706) (size 0.7) (drill 0.4) (layers "F.Cu" "B.Cu") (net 2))
 (via (at 123.698 52.705) (size 0.7) (drill 0.4) (layers "F.Cu" "B.Cu") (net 2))
 (via (at 123.571 56.134) (size 0.7) (drill 0.4) (layers "F.Cu" "B.Cu") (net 2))
 (via (at 131.826 49.403) (size 0.7) (drill 0.4) (layers "F.Cu" "B.Cu") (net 2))
 (segment (start 128.230999 41.997999) (end 127.381 41.148) (width 0.3) (layer "B.Cu") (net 2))
 (segment (start 131.191 42.418) (end 128.651 42.418) (width 0.3) (layer "B.Cu") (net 2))
 (segment (start 132.461 43.688) (end 131.191 42.418) (width 0.3) (layer "B.Cu") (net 2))
 (segment (start 128.651 42.418) (end 128.230999 41.997999) (width 0.3) (layer "B.Cu") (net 2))
 (segment (start 126.776 60.85) (end 126.776 62.357) (width 0.2) (layer "F.Cu") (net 5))
 (segment (start 129.286 58.072) (end 128.679 58.072) (width 0.2) (layer "F.Cu") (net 5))
 (segment (start 128.679 58.072) (end 126.873 59.878) (width 0.2) (layer "F.Cu") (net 5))
 (segment (start 126.873 60.753) (end 126.776 60.85) (width 0.2) (layer "F.Cu") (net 5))
 (segment (start 126.873 59.878) (end 126.873 60.753) (width 0.2) (layer "F.Cu") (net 5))
 (segment (start 130.556 57.023) (end 130.556 58.072) (width 0.2) (layer "F.Cu") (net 4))
 (segment (start 126.223 60.753) (end 126.223 59.197) (width 0.2) (layer "F.Cu") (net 4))
 (segment (start 128.778 56.642) (end 130.175 56.642) (width 0.2) (layer "F.Cu") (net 4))
 (segment (start 126.223 59.197) (end 128.778 56.642) (width 0.2) (layer "F.Cu") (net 4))
 (segment (start 130.175 56.642) (end 130.556 57.023) (width 0.2) (layer "F.Cu") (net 4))
 (segment (start 126.223 60.753) (end 126.223 61.371) (width 0.2) (layer "F.Cu") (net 4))
 (segment (start 126.223 61.371) (end 126.126 61.468) (width 0.2) (layer "F.Cu") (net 4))
 (via (at 126.126 61.468) (size 0.6) (drill 0.3) (layers "F.Cu" "B.Cu") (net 4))
 (segment (start 124.825 63.357) (end 126.126 63.357) (width 0.2) (layer "B.Cu") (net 4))
 (segment (start 124.714 61.849) (end 124.714 63.246) (width 0.2) (layer "B.Cu") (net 4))
 (segment (start 124.714 63.246) (end 124.825 63.357) (width 0.2) (layer "B.Cu") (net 4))
 (segment (start 125.095 61.468) (end 124.714 61.849) (width 0.2) (layer "B.Cu") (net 4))
 (segment (start 126.126 61.468) (end 125.095 61.468) (width 0.2) (layer "B.Cu") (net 4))
 (segment (start 128.651 42.418) (end 129.071001 41.997999) (width 0.2) (layer "F.Cu") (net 11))
 (segment (start 126.746 46.355) (end 128.651 44.45) (width 0.2) (layer "F.Cu") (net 11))
 (segment (start 124.310072 46.854072) (end 123.811 46.355) (width 0.2) (layer "F.Cu") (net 11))
 (segment (start 128.620121 48.833881) (end 126.289881 48.833881) (width 0.2) (layer "F.Cu") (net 11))
 (segment (start 129.071001 41.997999) (end 129.921 41.148) (width 0.2) (layer "F.Cu") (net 11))
 (segment (start 123.811 46.355) (end 126.746 46.355) (width 0.2) (layer "F.Cu") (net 11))
 (segment (start 131.826 52.672) (end 131.826 54.229) (width 0.2) (layer "F.Cu") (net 11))
 (segment (start 131.826 54.229) (end 131.699 54.356) (width 0.2) (layer "F.Cu") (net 11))
 (segment (start 128.651 44.45) (end 128.651 42.418) (width 0.2) (layer "F.Cu") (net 11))
 (segment (start 128.92012 49.13388) (end 128.620121 48.833881) (width 0.2) (layer "F.Cu") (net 11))
 (segment (start 126.289881 48.833881) (end 124.310072 46.854072) (width 0.2) (layer "F.Cu") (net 11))
 (via (at 128.92012 49.13388) (size 0.6) (drill 0.3) (layers "F.Cu" "B.Cu") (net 11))
 (via (at 131.699 54.356) (size 0.6) (drill 0.3) (layers "F.Cu" "B.Cu") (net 11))
 (segment (start 128.92012 51.57712) (end 128.92012 49.13388) (width 0.2) (layer "B.Cu") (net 11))
 (segment (start 131.699 54.356) (end 128.92012 51.57712) (width 0.2) (layer "B.Cu") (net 11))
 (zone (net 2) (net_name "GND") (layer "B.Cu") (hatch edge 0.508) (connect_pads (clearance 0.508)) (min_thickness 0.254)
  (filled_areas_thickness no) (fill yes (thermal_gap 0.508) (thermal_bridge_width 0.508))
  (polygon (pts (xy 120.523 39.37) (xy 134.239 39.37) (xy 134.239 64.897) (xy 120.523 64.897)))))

